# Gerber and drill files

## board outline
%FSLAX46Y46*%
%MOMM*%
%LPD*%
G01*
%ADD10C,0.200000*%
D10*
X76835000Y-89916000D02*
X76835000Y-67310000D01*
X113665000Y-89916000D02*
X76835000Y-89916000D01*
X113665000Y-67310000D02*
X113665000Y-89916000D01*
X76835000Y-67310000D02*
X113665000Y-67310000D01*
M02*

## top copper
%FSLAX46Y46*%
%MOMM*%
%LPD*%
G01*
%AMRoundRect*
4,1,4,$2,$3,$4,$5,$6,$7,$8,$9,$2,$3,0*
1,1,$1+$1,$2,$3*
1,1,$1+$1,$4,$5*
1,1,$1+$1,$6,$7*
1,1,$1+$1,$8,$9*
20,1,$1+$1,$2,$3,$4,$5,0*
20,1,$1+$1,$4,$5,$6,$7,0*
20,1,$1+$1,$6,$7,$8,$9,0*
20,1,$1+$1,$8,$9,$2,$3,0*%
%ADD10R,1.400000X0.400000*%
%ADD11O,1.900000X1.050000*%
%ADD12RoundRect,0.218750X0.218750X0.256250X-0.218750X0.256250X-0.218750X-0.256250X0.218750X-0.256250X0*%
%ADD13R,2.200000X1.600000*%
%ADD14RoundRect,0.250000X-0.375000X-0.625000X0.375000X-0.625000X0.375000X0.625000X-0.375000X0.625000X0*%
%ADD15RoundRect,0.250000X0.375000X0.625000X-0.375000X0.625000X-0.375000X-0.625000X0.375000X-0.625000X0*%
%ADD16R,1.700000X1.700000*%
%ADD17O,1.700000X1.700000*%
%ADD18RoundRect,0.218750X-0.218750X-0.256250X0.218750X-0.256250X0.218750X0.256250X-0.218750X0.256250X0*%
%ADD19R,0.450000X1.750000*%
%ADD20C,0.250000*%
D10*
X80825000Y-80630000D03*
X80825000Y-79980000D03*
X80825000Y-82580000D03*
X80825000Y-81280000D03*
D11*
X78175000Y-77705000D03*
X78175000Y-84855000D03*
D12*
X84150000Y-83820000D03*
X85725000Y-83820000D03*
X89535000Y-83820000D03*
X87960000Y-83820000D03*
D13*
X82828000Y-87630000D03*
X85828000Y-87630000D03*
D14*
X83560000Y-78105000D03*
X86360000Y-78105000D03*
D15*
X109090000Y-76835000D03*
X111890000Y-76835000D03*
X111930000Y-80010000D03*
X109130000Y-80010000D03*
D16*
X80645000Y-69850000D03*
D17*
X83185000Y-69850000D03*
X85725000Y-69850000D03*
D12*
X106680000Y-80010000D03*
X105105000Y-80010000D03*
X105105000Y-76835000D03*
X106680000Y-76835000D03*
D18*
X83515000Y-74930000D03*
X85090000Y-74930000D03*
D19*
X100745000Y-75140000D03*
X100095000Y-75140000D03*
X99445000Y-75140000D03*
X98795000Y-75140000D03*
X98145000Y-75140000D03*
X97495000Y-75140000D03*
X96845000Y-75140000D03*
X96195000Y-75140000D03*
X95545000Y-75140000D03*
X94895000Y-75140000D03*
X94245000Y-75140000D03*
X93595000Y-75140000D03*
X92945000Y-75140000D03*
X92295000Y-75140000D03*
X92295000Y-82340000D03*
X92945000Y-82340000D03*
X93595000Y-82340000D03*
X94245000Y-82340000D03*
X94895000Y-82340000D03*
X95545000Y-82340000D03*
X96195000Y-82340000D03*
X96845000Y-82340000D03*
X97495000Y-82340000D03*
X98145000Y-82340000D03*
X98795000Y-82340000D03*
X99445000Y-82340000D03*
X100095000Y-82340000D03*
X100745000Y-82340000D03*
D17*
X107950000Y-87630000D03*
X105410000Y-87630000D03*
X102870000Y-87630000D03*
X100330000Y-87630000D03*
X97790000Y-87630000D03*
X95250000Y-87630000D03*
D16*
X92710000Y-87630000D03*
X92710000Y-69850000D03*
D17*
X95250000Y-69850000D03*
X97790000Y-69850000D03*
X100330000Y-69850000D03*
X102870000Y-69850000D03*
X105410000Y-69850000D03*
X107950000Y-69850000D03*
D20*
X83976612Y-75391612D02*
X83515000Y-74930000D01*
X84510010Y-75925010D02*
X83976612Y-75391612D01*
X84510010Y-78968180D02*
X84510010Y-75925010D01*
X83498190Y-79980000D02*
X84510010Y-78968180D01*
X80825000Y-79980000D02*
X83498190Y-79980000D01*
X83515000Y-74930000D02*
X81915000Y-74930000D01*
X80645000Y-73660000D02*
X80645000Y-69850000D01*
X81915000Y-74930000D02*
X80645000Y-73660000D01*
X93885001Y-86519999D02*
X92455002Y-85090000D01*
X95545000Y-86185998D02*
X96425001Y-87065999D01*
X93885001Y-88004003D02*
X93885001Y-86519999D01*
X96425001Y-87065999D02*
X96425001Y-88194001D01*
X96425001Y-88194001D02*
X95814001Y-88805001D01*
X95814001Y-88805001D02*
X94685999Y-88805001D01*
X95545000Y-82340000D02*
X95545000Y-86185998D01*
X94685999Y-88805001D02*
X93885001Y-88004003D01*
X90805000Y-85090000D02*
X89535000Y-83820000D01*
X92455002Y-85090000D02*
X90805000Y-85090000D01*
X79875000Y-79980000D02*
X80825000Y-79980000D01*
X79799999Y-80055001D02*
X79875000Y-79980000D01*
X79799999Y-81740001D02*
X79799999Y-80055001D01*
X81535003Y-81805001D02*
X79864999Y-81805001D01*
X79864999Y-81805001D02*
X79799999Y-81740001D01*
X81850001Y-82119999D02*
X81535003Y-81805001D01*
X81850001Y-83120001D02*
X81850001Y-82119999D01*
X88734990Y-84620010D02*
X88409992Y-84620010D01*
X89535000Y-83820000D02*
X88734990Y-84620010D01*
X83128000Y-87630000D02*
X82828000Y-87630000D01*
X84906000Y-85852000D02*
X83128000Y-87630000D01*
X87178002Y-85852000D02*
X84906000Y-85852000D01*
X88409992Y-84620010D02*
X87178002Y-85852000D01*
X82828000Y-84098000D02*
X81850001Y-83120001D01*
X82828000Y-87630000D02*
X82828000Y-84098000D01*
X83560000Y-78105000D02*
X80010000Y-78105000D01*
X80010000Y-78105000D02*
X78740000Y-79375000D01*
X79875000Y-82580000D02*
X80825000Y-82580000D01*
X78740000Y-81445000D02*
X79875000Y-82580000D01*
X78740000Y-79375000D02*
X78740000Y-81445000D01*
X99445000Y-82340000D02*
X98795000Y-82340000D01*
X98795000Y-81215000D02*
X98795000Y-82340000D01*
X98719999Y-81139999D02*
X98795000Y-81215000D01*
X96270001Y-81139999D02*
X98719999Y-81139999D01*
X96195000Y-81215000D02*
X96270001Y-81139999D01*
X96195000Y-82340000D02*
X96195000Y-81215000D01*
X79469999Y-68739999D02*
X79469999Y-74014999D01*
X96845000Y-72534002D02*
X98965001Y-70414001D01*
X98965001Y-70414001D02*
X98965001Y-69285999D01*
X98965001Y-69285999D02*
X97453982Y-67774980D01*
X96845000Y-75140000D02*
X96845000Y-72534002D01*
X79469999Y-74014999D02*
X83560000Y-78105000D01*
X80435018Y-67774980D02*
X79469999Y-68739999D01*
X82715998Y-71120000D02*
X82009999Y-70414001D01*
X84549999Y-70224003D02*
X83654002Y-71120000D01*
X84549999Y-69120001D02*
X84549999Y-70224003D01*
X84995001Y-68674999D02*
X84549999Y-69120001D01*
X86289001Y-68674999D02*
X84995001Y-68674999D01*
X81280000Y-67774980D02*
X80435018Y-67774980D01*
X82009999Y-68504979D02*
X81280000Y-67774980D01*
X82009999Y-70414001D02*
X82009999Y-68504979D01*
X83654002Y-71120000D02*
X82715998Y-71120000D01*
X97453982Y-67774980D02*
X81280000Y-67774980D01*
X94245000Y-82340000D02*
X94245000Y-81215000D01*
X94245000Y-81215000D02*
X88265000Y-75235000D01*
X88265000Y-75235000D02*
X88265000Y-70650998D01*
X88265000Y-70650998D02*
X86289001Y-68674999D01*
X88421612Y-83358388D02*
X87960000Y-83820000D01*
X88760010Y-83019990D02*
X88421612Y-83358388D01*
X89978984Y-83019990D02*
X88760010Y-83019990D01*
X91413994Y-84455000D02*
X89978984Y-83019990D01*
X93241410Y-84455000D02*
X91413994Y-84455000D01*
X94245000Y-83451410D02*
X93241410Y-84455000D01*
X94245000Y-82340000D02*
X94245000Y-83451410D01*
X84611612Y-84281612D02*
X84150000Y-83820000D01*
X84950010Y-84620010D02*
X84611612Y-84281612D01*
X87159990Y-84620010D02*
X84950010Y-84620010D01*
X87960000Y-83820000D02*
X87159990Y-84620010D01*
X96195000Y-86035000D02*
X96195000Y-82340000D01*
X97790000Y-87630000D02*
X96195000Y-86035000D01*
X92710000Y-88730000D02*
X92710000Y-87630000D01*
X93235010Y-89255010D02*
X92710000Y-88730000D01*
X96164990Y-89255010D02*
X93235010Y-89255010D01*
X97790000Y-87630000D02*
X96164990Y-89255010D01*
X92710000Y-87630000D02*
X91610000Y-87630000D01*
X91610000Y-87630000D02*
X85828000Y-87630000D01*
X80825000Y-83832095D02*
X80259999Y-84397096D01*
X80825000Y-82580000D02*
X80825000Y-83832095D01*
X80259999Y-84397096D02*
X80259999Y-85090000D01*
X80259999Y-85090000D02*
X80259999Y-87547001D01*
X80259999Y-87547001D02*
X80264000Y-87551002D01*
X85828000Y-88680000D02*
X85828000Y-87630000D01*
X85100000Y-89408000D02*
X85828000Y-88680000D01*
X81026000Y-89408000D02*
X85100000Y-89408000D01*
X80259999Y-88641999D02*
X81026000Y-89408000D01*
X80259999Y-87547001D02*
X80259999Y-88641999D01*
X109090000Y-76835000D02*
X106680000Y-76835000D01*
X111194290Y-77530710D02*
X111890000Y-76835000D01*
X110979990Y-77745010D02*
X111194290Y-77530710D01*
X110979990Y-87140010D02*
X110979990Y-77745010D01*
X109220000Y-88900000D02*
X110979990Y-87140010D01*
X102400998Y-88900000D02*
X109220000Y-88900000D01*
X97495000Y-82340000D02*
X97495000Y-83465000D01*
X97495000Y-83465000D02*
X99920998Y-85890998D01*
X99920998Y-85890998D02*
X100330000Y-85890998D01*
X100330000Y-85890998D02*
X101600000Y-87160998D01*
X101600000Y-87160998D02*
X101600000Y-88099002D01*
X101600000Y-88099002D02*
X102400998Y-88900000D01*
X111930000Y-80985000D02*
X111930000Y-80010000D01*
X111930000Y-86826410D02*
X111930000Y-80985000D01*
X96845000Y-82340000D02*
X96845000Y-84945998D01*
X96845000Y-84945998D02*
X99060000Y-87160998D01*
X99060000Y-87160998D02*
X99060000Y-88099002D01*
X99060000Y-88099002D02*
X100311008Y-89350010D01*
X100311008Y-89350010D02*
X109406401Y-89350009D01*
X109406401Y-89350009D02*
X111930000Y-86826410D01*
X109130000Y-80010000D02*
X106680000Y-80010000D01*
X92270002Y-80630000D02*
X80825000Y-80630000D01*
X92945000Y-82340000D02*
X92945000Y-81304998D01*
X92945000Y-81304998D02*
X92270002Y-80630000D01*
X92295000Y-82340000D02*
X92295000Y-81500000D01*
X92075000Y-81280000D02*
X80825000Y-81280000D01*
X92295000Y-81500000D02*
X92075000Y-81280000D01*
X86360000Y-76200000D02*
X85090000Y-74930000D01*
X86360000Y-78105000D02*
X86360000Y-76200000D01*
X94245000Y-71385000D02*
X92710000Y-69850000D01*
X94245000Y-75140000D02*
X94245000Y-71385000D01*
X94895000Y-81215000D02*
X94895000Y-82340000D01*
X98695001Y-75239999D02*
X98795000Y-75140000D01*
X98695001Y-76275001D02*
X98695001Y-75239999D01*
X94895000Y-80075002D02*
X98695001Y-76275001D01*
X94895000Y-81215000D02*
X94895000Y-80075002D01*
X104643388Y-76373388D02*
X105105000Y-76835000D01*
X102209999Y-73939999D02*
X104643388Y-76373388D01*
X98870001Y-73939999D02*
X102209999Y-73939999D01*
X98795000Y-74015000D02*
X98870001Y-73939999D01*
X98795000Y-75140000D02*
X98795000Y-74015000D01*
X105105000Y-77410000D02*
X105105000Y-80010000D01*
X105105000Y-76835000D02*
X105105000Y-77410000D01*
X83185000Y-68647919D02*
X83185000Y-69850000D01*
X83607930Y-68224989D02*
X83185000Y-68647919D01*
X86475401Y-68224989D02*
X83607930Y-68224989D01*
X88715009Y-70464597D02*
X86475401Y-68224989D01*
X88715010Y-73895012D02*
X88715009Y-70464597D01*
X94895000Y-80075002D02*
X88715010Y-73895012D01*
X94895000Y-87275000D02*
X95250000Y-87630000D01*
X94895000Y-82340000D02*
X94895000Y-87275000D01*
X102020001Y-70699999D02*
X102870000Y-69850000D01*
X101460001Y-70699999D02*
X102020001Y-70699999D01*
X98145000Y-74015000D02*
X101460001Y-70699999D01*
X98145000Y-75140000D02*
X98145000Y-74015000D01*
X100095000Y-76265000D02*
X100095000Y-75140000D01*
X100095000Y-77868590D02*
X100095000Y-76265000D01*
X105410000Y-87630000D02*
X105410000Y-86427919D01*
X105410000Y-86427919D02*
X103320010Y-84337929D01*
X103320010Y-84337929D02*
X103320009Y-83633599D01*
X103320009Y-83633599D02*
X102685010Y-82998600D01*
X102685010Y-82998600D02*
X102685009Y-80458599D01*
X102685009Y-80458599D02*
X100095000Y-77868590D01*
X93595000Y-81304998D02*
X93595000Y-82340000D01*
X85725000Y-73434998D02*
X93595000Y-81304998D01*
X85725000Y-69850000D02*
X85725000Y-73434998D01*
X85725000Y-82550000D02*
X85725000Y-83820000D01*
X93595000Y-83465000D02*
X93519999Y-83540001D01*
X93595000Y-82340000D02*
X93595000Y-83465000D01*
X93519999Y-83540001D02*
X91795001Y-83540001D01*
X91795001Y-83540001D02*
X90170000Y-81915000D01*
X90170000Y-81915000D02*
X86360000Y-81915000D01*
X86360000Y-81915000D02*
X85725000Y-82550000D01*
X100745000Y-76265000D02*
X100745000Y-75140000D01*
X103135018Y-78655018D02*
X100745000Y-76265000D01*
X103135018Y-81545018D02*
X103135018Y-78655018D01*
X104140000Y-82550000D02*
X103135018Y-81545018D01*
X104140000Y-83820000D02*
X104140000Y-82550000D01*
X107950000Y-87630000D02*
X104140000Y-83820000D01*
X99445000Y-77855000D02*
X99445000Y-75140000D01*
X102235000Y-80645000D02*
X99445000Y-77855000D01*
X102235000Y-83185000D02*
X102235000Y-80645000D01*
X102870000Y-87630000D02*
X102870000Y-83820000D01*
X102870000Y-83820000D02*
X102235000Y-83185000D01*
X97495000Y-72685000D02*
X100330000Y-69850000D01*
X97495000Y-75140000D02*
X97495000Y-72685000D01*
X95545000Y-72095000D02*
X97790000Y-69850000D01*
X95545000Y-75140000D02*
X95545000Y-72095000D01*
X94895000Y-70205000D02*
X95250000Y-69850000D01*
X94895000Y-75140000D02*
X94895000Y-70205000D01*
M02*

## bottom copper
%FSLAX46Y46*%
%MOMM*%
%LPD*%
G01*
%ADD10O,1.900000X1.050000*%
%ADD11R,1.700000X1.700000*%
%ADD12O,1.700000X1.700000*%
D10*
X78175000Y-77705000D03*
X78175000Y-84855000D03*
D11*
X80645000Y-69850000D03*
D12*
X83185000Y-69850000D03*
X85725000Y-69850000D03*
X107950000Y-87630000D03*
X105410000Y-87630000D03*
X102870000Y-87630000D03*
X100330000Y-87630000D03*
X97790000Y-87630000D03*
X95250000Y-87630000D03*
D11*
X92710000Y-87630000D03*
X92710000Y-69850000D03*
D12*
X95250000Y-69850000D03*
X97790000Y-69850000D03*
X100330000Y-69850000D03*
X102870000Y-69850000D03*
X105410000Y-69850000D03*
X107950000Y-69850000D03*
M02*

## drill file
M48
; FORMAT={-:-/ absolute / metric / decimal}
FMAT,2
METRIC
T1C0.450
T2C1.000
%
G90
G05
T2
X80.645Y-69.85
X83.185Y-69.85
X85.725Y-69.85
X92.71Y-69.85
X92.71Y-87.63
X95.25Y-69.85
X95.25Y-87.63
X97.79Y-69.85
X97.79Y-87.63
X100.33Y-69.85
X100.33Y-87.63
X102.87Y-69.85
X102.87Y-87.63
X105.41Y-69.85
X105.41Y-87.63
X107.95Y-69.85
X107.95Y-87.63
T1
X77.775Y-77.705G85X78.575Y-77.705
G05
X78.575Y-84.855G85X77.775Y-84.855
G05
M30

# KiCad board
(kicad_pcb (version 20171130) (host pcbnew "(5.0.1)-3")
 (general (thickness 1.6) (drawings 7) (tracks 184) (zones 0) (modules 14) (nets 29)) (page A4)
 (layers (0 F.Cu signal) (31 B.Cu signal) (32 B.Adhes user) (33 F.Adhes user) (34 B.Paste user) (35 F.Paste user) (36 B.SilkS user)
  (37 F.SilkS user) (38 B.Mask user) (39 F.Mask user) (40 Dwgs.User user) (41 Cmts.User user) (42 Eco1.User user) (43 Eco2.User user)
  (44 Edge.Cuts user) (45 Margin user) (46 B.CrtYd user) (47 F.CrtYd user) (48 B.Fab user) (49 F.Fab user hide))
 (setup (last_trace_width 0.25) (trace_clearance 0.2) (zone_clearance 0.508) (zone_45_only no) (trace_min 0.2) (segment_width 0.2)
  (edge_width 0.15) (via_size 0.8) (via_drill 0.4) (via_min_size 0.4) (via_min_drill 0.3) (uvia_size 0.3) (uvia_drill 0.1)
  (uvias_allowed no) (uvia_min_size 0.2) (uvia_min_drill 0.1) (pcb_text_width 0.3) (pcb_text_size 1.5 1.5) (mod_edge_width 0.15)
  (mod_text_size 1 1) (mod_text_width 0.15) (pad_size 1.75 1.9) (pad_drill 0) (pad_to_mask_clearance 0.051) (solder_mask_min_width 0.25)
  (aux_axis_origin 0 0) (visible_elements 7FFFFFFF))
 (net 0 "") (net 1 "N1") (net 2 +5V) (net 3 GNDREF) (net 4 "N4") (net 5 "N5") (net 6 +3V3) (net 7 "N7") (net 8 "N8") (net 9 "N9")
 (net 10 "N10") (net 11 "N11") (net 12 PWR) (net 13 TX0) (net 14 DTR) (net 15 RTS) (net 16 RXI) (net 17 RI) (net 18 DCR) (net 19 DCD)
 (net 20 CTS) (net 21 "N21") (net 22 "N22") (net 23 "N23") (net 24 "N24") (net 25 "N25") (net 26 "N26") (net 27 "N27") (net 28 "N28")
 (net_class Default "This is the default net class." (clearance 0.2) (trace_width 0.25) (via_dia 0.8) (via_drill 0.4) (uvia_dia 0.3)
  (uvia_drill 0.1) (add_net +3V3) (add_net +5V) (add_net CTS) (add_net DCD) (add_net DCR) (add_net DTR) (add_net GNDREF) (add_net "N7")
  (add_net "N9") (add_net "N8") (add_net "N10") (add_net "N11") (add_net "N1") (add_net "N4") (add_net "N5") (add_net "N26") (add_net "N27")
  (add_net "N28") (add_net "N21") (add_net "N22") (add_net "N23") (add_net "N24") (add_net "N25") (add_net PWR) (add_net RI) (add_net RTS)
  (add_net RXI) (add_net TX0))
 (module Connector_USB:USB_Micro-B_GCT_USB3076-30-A (layer F.Cu) (at 79.375 81.28 270)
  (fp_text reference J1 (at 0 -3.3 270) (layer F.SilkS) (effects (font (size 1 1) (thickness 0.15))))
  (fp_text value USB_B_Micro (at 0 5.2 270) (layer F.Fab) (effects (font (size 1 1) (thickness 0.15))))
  (pad 2 smd rect (at -0.65 -1.45 270) (size 0.4 1.4) (layers F.Cu F.Paste F.Mask) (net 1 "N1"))
  (pad 1 smd rect (at -1.3 -1.45 270) (size 0.4 1.4) (layers F.Cu F.Paste F.Mask) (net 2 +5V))
  (pad 5 smd rect (at 1.3 -1.45 270) (size 0.4 1.4) (layers F.Cu F.Paste F.Mask) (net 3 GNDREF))
  (pad 3 smd rect (at 0 -1.45 270) (size 0.4 1.4) (layers F.Cu F.Paste F.Mask) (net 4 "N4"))
  (pad 6 thru_hole oval (at -3.575 1.2 90) (size 1.05 1.9) (drill oval 0.45 1.25) (layers *.Cu *.Mask) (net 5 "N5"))
  (pad 6 thru_hole oval (at 3.575 1.2 270) (size 1.05 1.9) (drill oval 0.45 1.25) (layers *.Cu *.Mask) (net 5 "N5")))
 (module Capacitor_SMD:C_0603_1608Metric (layer F.Cu) (at 84.9375 83.82 180)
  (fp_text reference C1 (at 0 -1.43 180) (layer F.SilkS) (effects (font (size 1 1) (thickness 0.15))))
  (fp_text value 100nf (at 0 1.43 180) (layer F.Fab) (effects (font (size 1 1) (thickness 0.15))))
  (pad 2 smd roundrect (at 0.7875 0 180) (size 0.875 0.95) (layers F.Cu F.Paste F.Mask) (roundrect_rratio 0.25) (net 3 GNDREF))
  (pad 1 smd roundrect (at -0.7875 0 180) (size 0.875 0.95) (layers F.Cu F.Paste F.Mask) (roundrect_rratio 0.25) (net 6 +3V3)))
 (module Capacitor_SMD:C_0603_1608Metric (layer F.Cu) (at 88.7475 83.82 180)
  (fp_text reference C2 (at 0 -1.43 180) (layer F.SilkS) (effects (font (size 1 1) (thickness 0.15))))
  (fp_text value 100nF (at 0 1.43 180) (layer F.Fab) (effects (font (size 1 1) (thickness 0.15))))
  (pad 1 smd roundrect (at -0.7875 0 180) (size 0.875 0.95) (layers F.Cu F.Paste F.Mask) (roundrect_rratio 0.25) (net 2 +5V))
  (pad 2 smd roundrect (at 0.7875 0 180) (size 0.875 0.95) (layers F.Cu F.Paste F.Mask) (roundrect_rratio 0.25) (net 3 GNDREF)))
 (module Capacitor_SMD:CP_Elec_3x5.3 (layer F.Cu) (at 84.328 87.63)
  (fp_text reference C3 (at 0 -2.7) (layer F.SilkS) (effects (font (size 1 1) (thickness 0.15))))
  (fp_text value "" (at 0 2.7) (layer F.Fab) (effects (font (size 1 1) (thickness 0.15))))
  (pad 1 smd rect (at -1.5 0) (size 2.2 1.6) (layers F.Cu F.Paste F.Mask) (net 2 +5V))
  (pad 2 smd rect (at 1.5 0) (size 2.2 1.6) (layers F.Cu F.Paste F.Mask) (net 3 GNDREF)))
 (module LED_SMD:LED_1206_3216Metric (layer F.Cu) (at 84.96 78.105)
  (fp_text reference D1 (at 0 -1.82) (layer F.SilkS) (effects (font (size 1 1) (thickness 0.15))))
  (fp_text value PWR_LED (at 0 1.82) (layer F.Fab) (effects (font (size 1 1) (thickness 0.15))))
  (pad 1 smd roundrect (at -1.4 0) (size 1.25 1.75) (layers F.Cu F.Paste F.Mask) (roundrect_rratio 0.2) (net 3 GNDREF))
  (pad 2 smd roundrect (at 1.4 0) (size 1.25 1.75) (layers F.Cu F.Paste F.Mask) (roundrect_rratio 0.2) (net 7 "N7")))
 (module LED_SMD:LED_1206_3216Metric (layer F.Cu) (at 110.49 76.835 180)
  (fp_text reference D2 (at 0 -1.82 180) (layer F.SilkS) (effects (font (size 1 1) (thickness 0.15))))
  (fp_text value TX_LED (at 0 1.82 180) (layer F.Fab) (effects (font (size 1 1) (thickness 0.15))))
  (pad 2 smd roundrect (at 1.4 0 180) (size 1.25 1.75) (layers F.Cu F.Paste F.Mask) (roundrect_rratio 0.2) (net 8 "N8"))
  (pad 1 smd roundrect (at -1.4 0 180) (size 1.25 1.75) (layers F.Cu F.Paste F.Mask) (roundrect_rratio 0.2) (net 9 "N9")))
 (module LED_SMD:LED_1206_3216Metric (layer F.Cu) (at 110.53 80.01 180)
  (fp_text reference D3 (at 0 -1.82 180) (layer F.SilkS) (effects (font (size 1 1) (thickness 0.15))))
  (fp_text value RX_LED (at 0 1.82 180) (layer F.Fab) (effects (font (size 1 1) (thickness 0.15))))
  (pad 1 smd roundrect (at -1.4 0 180) (size 1.25 1.75) (layers F.Cu F.Paste F.Mask) (roundrect_rratio 0.2) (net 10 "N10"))
  (pad 2 smd roundrect (at 1.4 0 180) (size 1.25 1.75) (layers F.Cu F.Paste F.Mask) (roundrect_rratio 0.2) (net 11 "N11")))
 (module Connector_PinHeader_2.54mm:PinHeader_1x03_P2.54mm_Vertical (layer F.Cu) (at 80.645 69.85 90)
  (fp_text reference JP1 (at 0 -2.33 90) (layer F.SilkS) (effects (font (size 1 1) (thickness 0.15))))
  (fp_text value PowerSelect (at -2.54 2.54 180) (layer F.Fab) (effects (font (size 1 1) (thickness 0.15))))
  (pad 1 thru_hole rect (at 0 0 90) (size 1.7 1.7) (drill 1) (layers *.Cu *.Mask) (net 2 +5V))
  (pad 2 thru_hole oval (at 0 2.54 90) (size 1.7 1.7) (drill 1) (layers *.Cu *.Mask) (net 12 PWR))
  (pad 3 thru_hole oval (at 0 5.08 90) (size 1.7 1.7) (drill 1) (layers *.Cu *.Mask) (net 6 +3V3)))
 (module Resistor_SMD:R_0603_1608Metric (layer F.Cu) (at 105.8925 80.01 180)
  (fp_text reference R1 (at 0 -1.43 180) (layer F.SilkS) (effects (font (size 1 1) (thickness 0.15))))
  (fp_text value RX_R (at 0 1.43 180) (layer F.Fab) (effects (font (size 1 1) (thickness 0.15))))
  (pad 1 smd roundrect (at -0.7875 0 180) (size 0.875 0.95) (layers F.Cu F.Paste F.Mask) (roundrect_rratio 0.25) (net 11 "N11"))
  (pad 2 smd roundrect (at 0.7875 0 180) (size 0.875 0.95) (layers F.Cu F.Paste F.Mask) (roundrect_rratio 0.25) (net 12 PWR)))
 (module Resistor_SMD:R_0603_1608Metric (layer F.Cu) (at 105.8925 76.835 180)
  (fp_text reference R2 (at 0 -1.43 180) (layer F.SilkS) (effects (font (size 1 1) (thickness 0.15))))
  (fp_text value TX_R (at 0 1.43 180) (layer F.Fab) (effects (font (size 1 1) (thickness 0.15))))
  (pad 2 smd roundrect (at 0.7875 0 180) (size 0.875 0.95) (layers F.Cu F.Paste F.Mask) (roundrect_rratio 0.25) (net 12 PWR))
  (pad 1 smd roundrect (at -0.7875 0 180) (size 0.875 0.95) (layers F.Cu F.Paste F.Mask) (roundrect_rratio 0.25) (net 8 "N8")))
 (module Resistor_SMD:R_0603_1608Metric (layer F.Cu) (at 84.3025 74.93)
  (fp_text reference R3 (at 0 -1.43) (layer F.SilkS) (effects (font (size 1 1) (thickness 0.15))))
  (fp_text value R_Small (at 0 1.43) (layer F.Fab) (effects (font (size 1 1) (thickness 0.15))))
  (pad 1 smd roundrect (at -0.7875 0) (size 0.875 0.95) (layers F.Cu F.Paste F.Mask) (roundrect_rratio 0.25) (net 2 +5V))
  (pad 2 smd roundrect (at 0.7875 0) (size 0.875 0.95) (layers F.Cu F.Paste F.Mask) (roundrect_rratio 0.25) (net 7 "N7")))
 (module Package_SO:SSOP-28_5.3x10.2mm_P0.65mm (layer F.Cu) (at 96.52 78.74 270)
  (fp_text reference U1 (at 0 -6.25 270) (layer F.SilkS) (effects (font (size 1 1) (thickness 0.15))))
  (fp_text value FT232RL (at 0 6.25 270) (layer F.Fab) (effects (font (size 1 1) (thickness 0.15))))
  (pad 1 smd rect (at -3.6 -4.225 270) (size 1.75 0.45) (layers F.Cu F.Paste F.Mask) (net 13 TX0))
  (pad 2 smd rect (at -3.6 -3.575 270) (size 1.75 0.45) (layers F.Cu F.Paste F.Mask) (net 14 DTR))
  (pad 3 smd rect (at -3.6 -2.925 270) (size 1.75 0.45) (layers F.Cu F.Paste F.Mask) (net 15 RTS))
  (pad 4 smd rect (at -3.6 -2.275 270) (size 1.75 0.45) (layers F.Cu F.Paste F.Mask) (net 12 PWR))
  (pad 5 smd rect (at -3.6 -1.625 270) (size 1.75 0.45) (layers F.Cu F.Paste F.Mask) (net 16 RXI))
  (pad 6 smd rect (at -3.6 -0.975 270) (size 1.75 0.45) (layers F.Cu F.Paste F.Mask) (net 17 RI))
  (pad 7 smd rect (at -3.6 -0.325 270) (size 1.75 0.45) (layers F.Cu F.Paste F.Mask) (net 3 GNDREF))
  (pad 8 smd rect (at -3.6 0.325 270) (size 1.75 0.45) (layers F.Cu F.Paste F.Mask))
  (pad 9 smd rect (at -3.6 0.975 270) (size 1.75 0.45) (layers F.Cu F.Paste F.Mask) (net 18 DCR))
  (pad 10 smd rect (at -3.6 1.625 270) (size 1.75 0.45) (layers F.Cu F.Paste F.Mask) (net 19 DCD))
  (pad 11 smd rect (at -3.6 2.275 270) (size 1.75 0.45) (layers F.Cu F.Paste F.Mask) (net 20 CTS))
  (pad 12 smd rect (at -3.6 2.925 270) (size 1.75 0.45) (layers F.Cu F.Paste F.Mask) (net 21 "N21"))
  (pad 13 smd rect (at -3.6 3.575 270) (size 1.75 0.45) (layers F.Cu F.Paste F.Mask) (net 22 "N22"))
  (pad 14 smd rect (at -3.6 4.225 270) (size 1.75 0.45) (layers F.Cu F.Paste F.Mask) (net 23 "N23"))
  (pad 15 smd rect (at 3.6 4.225 270) (size 1.75 0.45) (layers F.Cu F.Paste F.Mask) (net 4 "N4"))
  (pad 16 smd rect (at 3.6 3.575 270) (size 1.75 0.45) (layers F.Cu F.Paste F.Mask) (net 1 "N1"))
  (pad 17 smd rect (at 3.6 2.925 270) (size 1.75 0.45) (layers F.Cu F.Paste F.Mask) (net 6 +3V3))
  (pad 18 smd rect (at 3.6 2.275 270) (size 1.75 0.45) (layers F.Cu F.Paste F.Mask) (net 3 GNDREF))
  (pad 19 smd rect (at 3.6 1.625 270) (size 1.75 0.45) (layers F.Cu F.Paste F.Mask) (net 12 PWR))
  (pad 20 smd rect (at 3.6 0.975 270) (size 1.75 0.45) (layers F.Cu F.Paste F.Mask) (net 2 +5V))
  (pad 21 smd rect (at 3.6 0.325 270) (size 1.75 0.45) (layers F.Cu F.Paste F.Mask) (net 3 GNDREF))
  (pad 22 smd rect (at 3.6 -0.325 270) (size 1.75 0.45) (layers F.Cu F.Paste F.Mask) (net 10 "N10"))
  (pad 23 smd rect (at 3.6 -0.975 270) (size 1.75 0.45) (layers F.Cu F.Paste F.Mask) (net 9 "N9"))
  (pad 24 smd rect (at 3.6 -1.625 270) (size 1.75 0.45) (layers F.Cu F.Paste F.Mask))
  (pad 25 smd rect (at 3.6 -2.275 270) (size 1.75 0.45) (layers F.Cu F.Paste F.Mask) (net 3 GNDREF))
  (pad 26 smd rect (at 3.6 -2.925 270) (size 1.75 0.45) (layers F.Cu F.Paste F.Mask) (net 3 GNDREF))
  (pad 27 smd rect (at 3.6 -3.575 270) (size 1.75 0.45) (layers F.Cu F.Paste F.Mask) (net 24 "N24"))
  (pad 28 smd rect (at 3.6 -4.225 270) (size 1.75 0.45) (layers F.Cu F.Paste F.Mask) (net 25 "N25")))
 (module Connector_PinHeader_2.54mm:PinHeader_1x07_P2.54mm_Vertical (layer F.Cu) (at 92.71 87.63 90)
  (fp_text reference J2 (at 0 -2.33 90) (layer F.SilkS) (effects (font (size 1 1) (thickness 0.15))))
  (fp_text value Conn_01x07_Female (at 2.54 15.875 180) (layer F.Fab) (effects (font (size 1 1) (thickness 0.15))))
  (pad 7 thru_hole oval (at 0 15.24 90) (size 1.7 1.7) (drill 1) (layers *.Cu *.Mask) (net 13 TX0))
  (pad 6 thru_hole oval (at 0 12.7 90) (size 1.7 1.7) (drill 1) (layers *.Cu *.Mask) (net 14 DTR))
  (pad 5 thru_hole oval (at 0 10.16 90) (size 1.7 1.7) (drill 1) (layers *.Cu *.Mask) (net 15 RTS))
  (pad 4 thru_hole oval (at 0 7.62 90) (size 1.7 1.7) (drill 1) (layers *.Cu *.Mask) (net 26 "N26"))
  (pad 3 thru_hole oval (at 0 5.08 90) (size 1.7 1.7) (drill 1) (layers *.Cu *.Mask) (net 3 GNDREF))
  (pad 2 thru_hole oval (at 0 2.54 90) (size 1.7 1.7) (drill 1) (layers *.Cu *.Mask) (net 12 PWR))
  (pad 1 thru_hole rect (at 0 0 90) (size 1.7 1.7) (drill 1) (layers *.Cu *.Mask) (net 3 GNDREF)))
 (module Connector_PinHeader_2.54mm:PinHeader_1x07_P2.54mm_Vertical (layer F.Cu) (at 92.71 69.85 90)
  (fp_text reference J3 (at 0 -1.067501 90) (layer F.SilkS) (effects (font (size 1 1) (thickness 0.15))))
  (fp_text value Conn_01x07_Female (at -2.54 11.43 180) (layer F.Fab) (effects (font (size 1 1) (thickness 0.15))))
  (pad 1 thru_hole rect (at 0 0 90) (size 1.7 1.7) (drill 1) (layers *.Cu *.Mask) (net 20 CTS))
  (pad 2 thru_hole oval (at 0 2.54 90) (size 1.7 1.7) (drill 1) (layers *.Cu *.Mask) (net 19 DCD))
  (pad 3 thru_hole oval (at 0 5.08 90) (size 1.7 1.7) (drill 1) (layers *.Cu *.Mask) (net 18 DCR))
  (pad 4 thru_hole oval (at 0 7.62 90) (size 1.7 1.7) (drill 1) (layers *.Cu *.Mask) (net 17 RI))
  (pad 5 thru_hole oval (at 0 10.16 90) (size 1.7 1.7) (drill 1) (layers *.Cu *.Mask) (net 16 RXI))
  (pad 6 thru_hole oval (at 0 12.7 90) (size 1.7 1.7) (drill 1) (layers *.Cu *.Mask) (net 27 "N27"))
  (pad 7 thru_hole oval (at 0 15.24 90) (size 1.7 1.7) (drill 1) (layers *.Cu *.Mask) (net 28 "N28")))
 (gr_line (start 76.835 89.916) (end 76.835 67.31) (layer Edge.Cuts) (width 0.2))
 (gr_line (start 113.665 89.916) (end 76.835 89.916) (layer Edge.Cuts) (width 0.2))
 (gr_line (start 113.665 67.31) (end 113.665 89.916) (layer Edge.Cuts) (width 0.2))
 (gr_line (start 76.835 67.31) (end 113.665 67.31) (layer Edge.Cuts) (width 0.2))
 (segment (start 83.976612 75.391612) (end 83.515 74.93) (width 0.25) (layer F.Cu) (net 2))
 (segment (start 84.51001 75.92501) (end 83.976612 75.391612) (width 0.25) (layer F.Cu) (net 2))
 (segment (start 84.51001 78.96818) (end 84.51001 75.92501) (width 0.25) (layer F.Cu) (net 2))
 (segment (start 83.49819 79.98) (end 84.51001 78.96818) (width 0.25) (layer F.Cu) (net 2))
 (segment (start 80.825 79.98) (end 83.49819 79.98) (width 0.25) (layer F.Cu) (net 2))
 (segment (start 83.515 74.93) (end 81.915 74.93) (width 0.25) (layer F.Cu) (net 2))
 (segment (start 80.645 73.66) (end 80.645 69.85) (width 0.25) (layer F.Cu) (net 2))
 (segment (start 81.915 74.93) (end 80.645 73.66) (width 0.25) (layer F.Cu) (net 2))
 (segment (start 93.885001 86.519999) (end 92.455002 85.09) (width 0.25) (layer F.Cu) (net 2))
 (segment (start 95.545 86.185998) (end 96.425001 87.065999) (width 0.25) (layer F.Cu) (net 2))
 (segment (start 93.885001 88.004003) (end 93.885001 86.519999) (width 0.25) (layer F.Cu) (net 2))
 (segment (start 96.425001 87.065999) (end 96.425001 88.194001) (width 0.25) (layer F.Cu) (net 2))
 (segment (start 96.425001 88.194001) (end 95.814001 88.805001) (width 0.25) (layer F.Cu) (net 2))
 (segment (start 95.814001 88.805001) (end 94.685999 88.805001) (width 0.25) (layer F.Cu) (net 2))
 (segment (start 95.545 82.34) (end 95.545 86.185998) (width 0.25) (layer F.Cu) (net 2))
 (segment (start 94.685999 88.805001) (end 93.885001 88.004003) (width 0.25) (layer F.Cu) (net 2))
 (segment (start 90.805 85.09) (end 89.535 83.82) (width 0.25) (layer F.Cu) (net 2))
 (segment (start 92.455002 85.09) (end 90.805 85.09) (width 0.25) (layer F.Cu) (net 2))
 (segment (start 79.875 79.98) (end 80.825 79.98) (width 0.25) (layer F.Cu) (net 2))
 (segment (start 79.799999 80.055001) (end 79.875 79.98) (width 0.25) (layer F.Cu) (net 2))
 (segment (start 79.799999 81.740001) (end 79.799999 80.055001) (width 0.25) (layer F.Cu) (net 2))
 (segment (start 81.535003 81.805001) (end 79.864999 81.805001) (width 0.25) (layer F.Cu) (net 2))
 (segment (start 79.864999 81.805001) (end 79.799999 81.740001) (width 0.25) (layer F.Cu) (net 2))
 (segment (start 81.850001 82.119999) (end 81.535003 81.805001) (width 0.25) (layer F.Cu) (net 2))
 (segment (start 81.850001 83.120001) (end 81.850001 82.119999) (width 0.25) (layer F.Cu) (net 2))
 (segment (start 88.73499 84.62001) (end 88.409992 84.62001) (width 0.25) (layer F.Cu) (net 2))
 (segment (start 89.535 83.82) (end 88.73499 84.62001) (width 0.25) (layer F.Cu) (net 2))
 (segment (start 83.128 87.63) (end 82.828 87.63) (width 0.25) (layer F.Cu) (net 2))
 (segment (start 84.906 85.852) (end 83.128 87.63) (width 0.25) (layer F.Cu) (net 2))
 (segment (start 87.178002 85.852) (end 84.906 85.852) (width 0.25) (layer F.Cu) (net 2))
 (segment (start 88.409992 84.62001) (end 87.178002 85.852) (width 0.25) (layer F.Cu) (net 2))
 (segment (start 82.828 84.098) (end 81.850001 83.120001) (width 0.25) (layer F.Cu) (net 2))
 (segment (start 82.828 87.63) (end 82.828 84.098) (width 0.25) (layer F.Cu) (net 2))
 (segment (start 83.56 78.105) (end 80.01 78.105) (width 0.25) (layer F.Cu) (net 3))
 (segment (start 80.01 78.105) (end 78.74 79.375) (width 0.25) (layer F.Cu) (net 3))
 (segment (start 79.875 82.58) (end 80.825 82.58) (width 0.25) (layer F.Cu) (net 3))
 (segment (start 78.74 81.445) (end 79.875 82.58) (width 0.25) (layer F.Cu) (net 3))
 (segment (start 78.74 79.375) (end 78.74 81.445) (width 0.25) (layer F.Cu) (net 3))
 (segment (start 99.445 82.34) (end 98.795 82.34) (width 0.25) (layer F.Cu) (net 3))
 (segment (start 98.795 81.215) (end 98.795 82.34) (width 0.25) (layer F.Cu) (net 3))
 (segment (start 98.719999 81.139999) (end 98.795 81.215) (width 0.25) (layer F.Cu) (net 3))
 (segment (start 96.270001 81.139999) (end 98.719999 81.139999) (width 0.25) (layer F.Cu) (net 3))
 (segment (start 96.195 81.215) (end 96.270001 81.139999) (width 0.25) (layer F.Cu) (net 3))
 (segment (start 96.195 82.34) (end 96.195 81.215) (width 0.25) (layer F.Cu) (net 3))
 (segment (start 79.469999 68.739999) (end 79.469999 74.014999) (width 0.25) (layer F.Cu) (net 3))
 (segment (start 96.845 72.534002) (end 98.965001 70.414001) (width 0.25) (layer F.Cu) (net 3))
 (segment (start 98.965001 70.414001) (end 98.965001 69.285999) (width 0.25) (layer F.Cu) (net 3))
 (segment (start 98.965001 69.285999) (end 97.453982 67.77498) (width 0.25) (layer F.Cu) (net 3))
 (segment (start 96.845 75.14) (end 96.845 72.534002) (width 0.25) (layer F.Cu) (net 3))
 (segment (start 79.469999 74.014999) (end 83.56 78.105) (width 0.25) (layer F.Cu) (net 3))
 (segment (start 80.435018 67.77498) (end 79.469999 68.739999) (width 0.25) (layer F.Cu) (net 3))
 (segment (start 82.715998 71.12) (end 82.009999 70.414001) (width 0.25) (layer F.Cu) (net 3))
 (segment (start 84.549999 70.224003) (end 83.654002 71.12) (width 0.25) (layer F.Cu) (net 3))
 (segment (start 84.549999 69.120001) (end 84.549999 70.224003) (width 0.25) (layer F.Cu) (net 3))
 (segment (start 84.995001 68.674999) (end 84.549999 69.120001) (width 0.25) (layer F.Cu) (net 3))
 (segment (start 86.289001 68.674999) (end 84.995001 68.674999) (width 0.25) (layer F.Cu) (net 3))
 (segment (start 81.28 67.77498) (end 80.435018 67.77498) (width 0.25) (layer F.Cu) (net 3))
 (segment (start 82.009999 68.504979) (end 81.28 67.77498) (width 0.25) (layer F.Cu) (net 3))
 (segment (start 82.009999 70.414001) (end 82.009999 68.504979) (width 0.25) (layer F.Cu) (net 3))
 (segment (start 83.654002 71.12) (end 82.715998 71.12) (width 0.25) (layer F.Cu) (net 3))
 (segment (start 97.453982 67.77498) (end 81.28 67.77498) (width 0.25) (layer F.Cu) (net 3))
 (segment (start 94.245 82.34) (end 94.245 81.215) (width 0.25) (layer F.Cu) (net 3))
 (segment (start 94.245 81.215) (end 88.265 75.235) (width 0.25) (layer F.Cu) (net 3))
 (segment (start 88.265 75.235) (end 88.265 70.650998) (width 0.25) (layer F.Cu) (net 3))
 (segment (start 88.265 70.650998) (end 86.289001 68.674999) (width 0.25) (layer F.Cu) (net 3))
 (segment (start 88.421612 83.358388) (end 87.96 83.82) (width 0.25) (layer F.Cu) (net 3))
 (segment (start 88.76001 83.01999) (end 88.421612 83.358388) (width 0.25) (layer F.Cu) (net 3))
 (segment (start 89.978984 83.01999) (end 88.76001 83.01999) (width 0.25) (layer F.Cu) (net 3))
 (segment (start 91.413994 84.455) (end 89.978984 83.01999) (width 0.25) (layer F.Cu) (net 3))
 (segment (start 93.24141 84.455) (end 91.413994 84.455) (width 0.25) (layer F.Cu) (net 3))
 (segment (start 94.245 83.45141) (end 93.24141 84.455) (width 0.25) (layer F.Cu) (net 3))
 (segment (start 94.245 82.34) (end 94.245 83.45141) (width 0.25) (layer F.Cu) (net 3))
 (segment (start 84.611612 84.281612) (end 84.15 83.82) (width 0.25) (layer F.Cu) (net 3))
 (segment (start 84.95001 84.62001) (end 84.611612 84.281612) (width 0.25) (layer F.Cu) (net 3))
 (segment (start 87.15999 84.62001) (end 84.95001 84.62001) (width 0.25) (layer F.Cu) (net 3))
 (segment (start 87.96 83.82) (end 87.15999 84.62001) (width 0.25) (layer F.Cu) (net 3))
 (segment (start 96.195 86.035) (end 96.195 82.34) (width 0.25) (layer F.Cu) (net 3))
 (segment (start 97.79 87.63) (end 96.195 86.035) (width 0.25) (layer F.Cu) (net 3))
 (segment (start 92.71 88.73) (end 92.71 87.63) (width 0.25) (layer F.Cu) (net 3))
 (segment (start 93.23501 89.25501) (end 92.71 88.73) (width 0.25) (layer F.Cu) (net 3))
 (segment (start 96.16499 89.25501) (end 93.23501 89.25501) (width 0.25) (layer F.Cu) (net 3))
 (segment (start 97.79 87.63) (end 96.16499 89.25501) (width 0.25) (layer F.Cu) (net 3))
 (segment (start 92.71 87.63) (end 91.61 87.63) (width 0.25) (layer F.Cu) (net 3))
 (segment (start 91.61 87.63) (end 85.828 87.63) (width 0.25) (layer F.Cu) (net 3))
 (segment (start 80.825 83.832095) (end 80.259999 84.397096) (width 0.25) (layer F.Cu) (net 3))
 (segment (start 80.825 82.58) (end 80.825 83.832095) (width 0.25) (layer F.Cu) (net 3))
 (segment (start 80.259999 84.397096) (end 80.259999 85.09) (width 0.25) (layer F.Cu) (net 3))
 (segment (start 80.259999 85.09) (end 80.259999 87.547001) (width 0.25) (layer F.Cu) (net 3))
 (segment (start 80.259999 87.547001) (end 80.264 87.551002) (width 0.25) (layer F.Cu) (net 3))
 (segment (start 85.828 88.68) (end 85.828 87.63) (width 0.25) (layer F.Cu) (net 3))
 (segment (start 85.1 89.408) (end 85.828 88.68) (width 0.25) (layer F.Cu) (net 3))
 (segment (start 81.026 89.408) (end 85.1 89.408) (width 0.25) (layer F.Cu) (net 3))
 (segment (start 80.259999 88.641999) (end 81.026 89.408) (width 0.25) (layer F.Cu) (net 3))
 (segment (start 80.259999 87.547001) (end 80.259999 88.641999) (width 0.25) (layer F.Cu) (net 3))
 (segment (start 109.09 76.835) (end 106.68 76.835) (width 0.25) (layer F.Cu) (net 8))
 (segment (start 111.19429 77.53071) (end 111.89 76.835) (width 0.25) (layer F.Cu) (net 9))
 (segment (start 110.97999 77.74501) (end 111.19429 77.53071) (width 0.25) (layer F.Cu) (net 9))
 (segment (start 110.97999 87.14001) (end 110.97999 77.74501) (width 0.25) (layer F.Cu) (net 9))
 (segment (start 109.22 88.9) (end 110.97999 87.14001) (width 0.25) (layer F.Cu) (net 9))
 (segment (start 102.400998 88.9) (end 109.22 88.9) (width 0.25) (layer F.Cu) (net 9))
 (segment (start 97.495 82.34) (end 97.495 83.465) (width 0.25) (layer F.Cu) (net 9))
 (segment (start 97.495 83.465) (end 99.920998 85.890998) (width 0.25) (layer F.Cu) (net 9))
 (segment (start 99.920998 85.890998) (end 100.33 85.890998) (width 0.25) (layer F.Cu) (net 9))
 (segment (start 100.33 85.890998) (end 101.6 87.160998) (width 0.25) (layer F.Cu) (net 9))
 (segment (start 101.6 87.160998) (end 101.6 88.099002) (width 0.25) (layer F.Cu) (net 9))
 (segment (start 101.6 88.099002) (end 102.400998 88.9) (width 0.25) (layer F.Cu) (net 9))
 (segment (start 111.93 80.985) (end 111.93 80.01) (width 0.25) (layer F.Cu) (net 10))
 (segment (start 111.93 86.82641) (end 111.93 80.985) (width 0.25) (layer F.Cu) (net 10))
 (segment (start 96.845 82.34) (end 96.845 84.945998) (width 0.25) (layer F.Cu) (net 10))
 (segment (start 96.845 84.945998) (end 99.06 87.160998) (width 0.25) (layer F.Cu) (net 10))
 (segment (start 99.06 87.160998) (end 99.06 88.099002) (width 0.25) (layer F.Cu) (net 10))
 (segment (start 99.06 88.099002) (end 100.311008 89.35001) (width 0.25) (layer F.Cu) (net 10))
 (segment (start 100.311008 89.35001) (end 109.406401 89.350009) (width 0.25) (layer F.Cu) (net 10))
 (segment (start 109.406401 89.350009) (end 111.93 86.82641) (width 0.25) (layer F.Cu) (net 10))
 (segment (start 109.13 80.01) (end 106.68 80.01) (width 0.25) (layer F.Cu) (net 11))
 (segment (start 92.270002 80.63) (end 80.825 80.63) (width 0.25) (layer F.Cu) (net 1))
 (segment (start 92.945 82.34) (end 92.945 81.304998) (width 0.25) (layer F.Cu) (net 1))
 (segment (start 92.945 81.304998) (end 92.270002 80.63) (width 0.25) (layer F.Cu) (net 1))
 (segment (start 92.295 82.34) (end 92.295 81.5) (width 0.25) (layer F.Cu) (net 4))
 (segment (start 92.075 81.28) (end 80.825 81.28) (width 0.25) (layer F.Cu) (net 4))
 (segment (start 92.295 81.5) (end 92.075 81.28) (width 0.25) (layer F.Cu) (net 4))
 (segment (start 86.36 76.2) (end 85.09 74.93) (width 0.25) (layer F.Cu) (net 7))
 (segment (start 86.36 78.105) (end 86.36 76.2) (width 0.25) (layer F.Cu) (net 7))
 (segment (start 94.245 71.385) (end 92.71 69.85) (width 0.25) (layer F.Cu) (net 20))
 (segment (start 94.245 75.14) (end 94.245 71.385) (width 0.25) (layer F.Cu) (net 20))
 (segment (start 94.895 81.215) (end 94.895 82.34) (width 0.25) (layer F.Cu) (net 12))
 (segment (start 98.695001 75.239999) (end 98.795 75.14) (width 0.25) (layer F.Cu) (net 12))
 (segment (start 98.695001 76.275001) (end 98.695001 75.239999) (width 0.25) (layer F.Cu) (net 12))
 (segment (start 94.895 80.075002) (end 98.695001 76.275001) (width 0.25) (layer F.Cu) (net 12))
 (segment (start 94.895 81.215) (end 94.895 80.075002) (width 0.25) (layer F.Cu) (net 12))
 (segment (start 104.643388 76.373388) (end 105.105 76.835) (width 0.25) (layer F.Cu) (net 12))
 (segment (start 102.209999 73.939999) (end 104.643388 76.373388) (width 0.25) (layer F.Cu) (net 12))
 (segment (start 98.870001 73.939999) (end 102.209999 73.939999) (width 0.25) (layer F.Cu) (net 12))
 (segment (start 98.795 74.015) (end 98.870001 73.939999) (width 0.25) (layer F.Cu) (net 12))
 (segment (start 98.795 75.14) (end 98.795 74.015) (width 0.25) (layer F.Cu) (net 12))
 (segment (start 105.105 77.41) (end 105.105 80.01) (width 0.25) (layer F.Cu) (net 12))
 (segment (start 105.105 76.835) (end 105.105 77.41) (width 0.25) (layer F.Cu) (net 12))
 (segment (start 83.185 68.647919) (end 83.185 69.85) (width 0.25) (layer F.Cu) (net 12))
 (segment (start 83.60793 68.224989) (end 83.185 68.647919) (width 0.25) (layer F.Cu) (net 12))
 (segment (start 86.475401 68.224989) (end 83.60793 68.224989) (width 0.25) (layer F.Cu) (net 12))
 (segment (start 88.715009 70.464597) (end 86.475401 68.224989) (width 0.25) (layer F.Cu) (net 12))
 (segment (start 88.71501 73.895012) (end 88.715009 70.464597) (width 0.25) (layer F.Cu) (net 12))
 (segment (start 94.895 80.075002) (end 88.71501 73.895012) (width 0.25) (layer F.Cu) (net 12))
 (segment (start 94.895 87.275) (end 95.25 87.63) (width 0.25) (layer F.Cu) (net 12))
 (segment (start 94.895 82.34) (end 94.895 87.275) (width 0.25) (layer F.Cu) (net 12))
 (segment (start 102.020001 70.699999) (end 102.87 69.85) (width 0.25) (layer F.Cu) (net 16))
 (segment (start 101.460001 70.699999) (end 102.020001 70.699999) (width 0.25) (layer F.Cu) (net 16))
 (segment (start 98.145 74.015) (end 101.460001 70.699999) (width 0.25) (layer F.Cu) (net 16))
 (segment (start 98.145 75.14) (end 98.145 74.015) (width 0.25) (layer F.Cu) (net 16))
 (segment (start 100.095 76.265) (end 100.095 75.14) (width 0.25) (layer F.Cu) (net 14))
 (segment (start 100.095 77.86859) (end 100.095 76.265) (width 0.25) (layer F.Cu) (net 14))
 (segment (start 105.41 87.63) (end 105.41 86.427919) (width 0.25) (layer F.Cu) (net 14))
 (segment (start 105.41 86.427919) (end 103.32001 84.337929) (width 0.25) (layer F.Cu) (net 14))
 (segment (start 103.32001 84.337929) (end 103.320009 83.633599) (width 0.25) (layer F.Cu) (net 14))
 (segment (start 103.320009 83.633599) (end 102.68501 82.9986) (width 0.25) (layer F.Cu) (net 14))
 (segment (start 102.68501 82.9986) (end 102.685009 80.458599) (width 0.25) (layer F.Cu) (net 14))
 (segment (start 102.685009 80.458599) (end 100.095 77.86859) (width 0.25) (layer F.Cu) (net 14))
 (segment (start 93.595 81.304998) (end 93.595 82.34) (width 0.25) (layer F.Cu) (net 6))
 (segment (start 85.725 73.434998) (end 93.595 81.304998) (width 0.25) (layer F.Cu) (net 6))
 (segment (start 85.725 69.85) (end 85.725 73.434998) (width 0.25) (layer F.Cu) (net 6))
 (segment (start 85.725 82.55) (end 85.725 83.82) (width 0.25) (layer F.Cu) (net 6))
 (segment (start 93.595 83.465) (end 93.519999 83.540001) (width 0.25) (layer F.Cu) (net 6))
 (segment (start 93.595 82.34) (end 93.595 83.465) (width 0.25) (layer F.Cu) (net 6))
 (segment (start 93.519999 83.540001) (end 91.795001 83.540001) (width 0.25) (layer F.Cu) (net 6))
 (segment (start 91.795001 83.540001) (end 90.17 81.915) (width 0.25) (layer F.Cu) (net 6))
 (segment (start 90.17 81.915) (end 86.36 81.915) (width 0.25) (layer F.Cu) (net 6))
 (segment (start 86.36 81.915) (end 85.725 82.55) (width 0.25) (layer F.Cu) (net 6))
 (segment (start 100.745 76.265) (end 100.745 75.14) (width 0.25) (layer F.Cu) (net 13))
 (segment (start 103.135018 78.655018) (end 100.745 76.265) (width 0.25) (layer F.Cu) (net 13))
 (segment (start 103.135018 81.545018) (end 103.135018 78.655018) (width 0.25) (layer F.Cu) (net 13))
 (segment (start 104.14 82.55) (end 103.135018 81.545018) (width 0.25) (layer F.Cu) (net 13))
 (segment (start 104.14 83.82) (end 104.14 82.55) (width 0.25) (layer F.Cu) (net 13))
 (segment (start 107.95 87.63) (end 104.14 83.82) (width 0.25) (layer F.Cu) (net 13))
 (segment (start 99.445 77.855) (end 99.445 75.14) (width 0.25) (layer F.Cu) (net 15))
 (segment (start 102.235 80.645) (end 99.445 77.855) (width 0.25) (layer F.Cu) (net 15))
 (segment (start 102.235 83.185) (end 102.235 80.645) (width 0.25) (layer F.Cu) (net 15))
 (segment (start 102.87 87.63) (end 102.87 83.82) (width 0.25) (layer F.Cu) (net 15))
 (segment (start 102.87 83.82) (end 102.235 83.185) (width 0.25) (layer F.Cu) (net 15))
 (segment (start 97.495 72.685) (end 100.33 69.85) (width 0.25) (layer F.Cu) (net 17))
 (segment (start 97.495 75.14) (end 97.495 72.685) (width 0.25) (layer F.Cu) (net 17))
 (segment (start 95.545 72.095) (end 97.79 69.85) (width 0.25) (layer F.Cu) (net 18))
 (segment (start 95.545 75.14) (end 95.545 72.095) (width 0.25) (layer F.Cu) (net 18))
 (segment (start 94.895 70.205) (end 95.25 69.85) (width 0.25) (layer F.Cu) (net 19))
 (segment (start 94.895 75.14) (end 94.895 70.205) (width 0.25) (layer F.Cu) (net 19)))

